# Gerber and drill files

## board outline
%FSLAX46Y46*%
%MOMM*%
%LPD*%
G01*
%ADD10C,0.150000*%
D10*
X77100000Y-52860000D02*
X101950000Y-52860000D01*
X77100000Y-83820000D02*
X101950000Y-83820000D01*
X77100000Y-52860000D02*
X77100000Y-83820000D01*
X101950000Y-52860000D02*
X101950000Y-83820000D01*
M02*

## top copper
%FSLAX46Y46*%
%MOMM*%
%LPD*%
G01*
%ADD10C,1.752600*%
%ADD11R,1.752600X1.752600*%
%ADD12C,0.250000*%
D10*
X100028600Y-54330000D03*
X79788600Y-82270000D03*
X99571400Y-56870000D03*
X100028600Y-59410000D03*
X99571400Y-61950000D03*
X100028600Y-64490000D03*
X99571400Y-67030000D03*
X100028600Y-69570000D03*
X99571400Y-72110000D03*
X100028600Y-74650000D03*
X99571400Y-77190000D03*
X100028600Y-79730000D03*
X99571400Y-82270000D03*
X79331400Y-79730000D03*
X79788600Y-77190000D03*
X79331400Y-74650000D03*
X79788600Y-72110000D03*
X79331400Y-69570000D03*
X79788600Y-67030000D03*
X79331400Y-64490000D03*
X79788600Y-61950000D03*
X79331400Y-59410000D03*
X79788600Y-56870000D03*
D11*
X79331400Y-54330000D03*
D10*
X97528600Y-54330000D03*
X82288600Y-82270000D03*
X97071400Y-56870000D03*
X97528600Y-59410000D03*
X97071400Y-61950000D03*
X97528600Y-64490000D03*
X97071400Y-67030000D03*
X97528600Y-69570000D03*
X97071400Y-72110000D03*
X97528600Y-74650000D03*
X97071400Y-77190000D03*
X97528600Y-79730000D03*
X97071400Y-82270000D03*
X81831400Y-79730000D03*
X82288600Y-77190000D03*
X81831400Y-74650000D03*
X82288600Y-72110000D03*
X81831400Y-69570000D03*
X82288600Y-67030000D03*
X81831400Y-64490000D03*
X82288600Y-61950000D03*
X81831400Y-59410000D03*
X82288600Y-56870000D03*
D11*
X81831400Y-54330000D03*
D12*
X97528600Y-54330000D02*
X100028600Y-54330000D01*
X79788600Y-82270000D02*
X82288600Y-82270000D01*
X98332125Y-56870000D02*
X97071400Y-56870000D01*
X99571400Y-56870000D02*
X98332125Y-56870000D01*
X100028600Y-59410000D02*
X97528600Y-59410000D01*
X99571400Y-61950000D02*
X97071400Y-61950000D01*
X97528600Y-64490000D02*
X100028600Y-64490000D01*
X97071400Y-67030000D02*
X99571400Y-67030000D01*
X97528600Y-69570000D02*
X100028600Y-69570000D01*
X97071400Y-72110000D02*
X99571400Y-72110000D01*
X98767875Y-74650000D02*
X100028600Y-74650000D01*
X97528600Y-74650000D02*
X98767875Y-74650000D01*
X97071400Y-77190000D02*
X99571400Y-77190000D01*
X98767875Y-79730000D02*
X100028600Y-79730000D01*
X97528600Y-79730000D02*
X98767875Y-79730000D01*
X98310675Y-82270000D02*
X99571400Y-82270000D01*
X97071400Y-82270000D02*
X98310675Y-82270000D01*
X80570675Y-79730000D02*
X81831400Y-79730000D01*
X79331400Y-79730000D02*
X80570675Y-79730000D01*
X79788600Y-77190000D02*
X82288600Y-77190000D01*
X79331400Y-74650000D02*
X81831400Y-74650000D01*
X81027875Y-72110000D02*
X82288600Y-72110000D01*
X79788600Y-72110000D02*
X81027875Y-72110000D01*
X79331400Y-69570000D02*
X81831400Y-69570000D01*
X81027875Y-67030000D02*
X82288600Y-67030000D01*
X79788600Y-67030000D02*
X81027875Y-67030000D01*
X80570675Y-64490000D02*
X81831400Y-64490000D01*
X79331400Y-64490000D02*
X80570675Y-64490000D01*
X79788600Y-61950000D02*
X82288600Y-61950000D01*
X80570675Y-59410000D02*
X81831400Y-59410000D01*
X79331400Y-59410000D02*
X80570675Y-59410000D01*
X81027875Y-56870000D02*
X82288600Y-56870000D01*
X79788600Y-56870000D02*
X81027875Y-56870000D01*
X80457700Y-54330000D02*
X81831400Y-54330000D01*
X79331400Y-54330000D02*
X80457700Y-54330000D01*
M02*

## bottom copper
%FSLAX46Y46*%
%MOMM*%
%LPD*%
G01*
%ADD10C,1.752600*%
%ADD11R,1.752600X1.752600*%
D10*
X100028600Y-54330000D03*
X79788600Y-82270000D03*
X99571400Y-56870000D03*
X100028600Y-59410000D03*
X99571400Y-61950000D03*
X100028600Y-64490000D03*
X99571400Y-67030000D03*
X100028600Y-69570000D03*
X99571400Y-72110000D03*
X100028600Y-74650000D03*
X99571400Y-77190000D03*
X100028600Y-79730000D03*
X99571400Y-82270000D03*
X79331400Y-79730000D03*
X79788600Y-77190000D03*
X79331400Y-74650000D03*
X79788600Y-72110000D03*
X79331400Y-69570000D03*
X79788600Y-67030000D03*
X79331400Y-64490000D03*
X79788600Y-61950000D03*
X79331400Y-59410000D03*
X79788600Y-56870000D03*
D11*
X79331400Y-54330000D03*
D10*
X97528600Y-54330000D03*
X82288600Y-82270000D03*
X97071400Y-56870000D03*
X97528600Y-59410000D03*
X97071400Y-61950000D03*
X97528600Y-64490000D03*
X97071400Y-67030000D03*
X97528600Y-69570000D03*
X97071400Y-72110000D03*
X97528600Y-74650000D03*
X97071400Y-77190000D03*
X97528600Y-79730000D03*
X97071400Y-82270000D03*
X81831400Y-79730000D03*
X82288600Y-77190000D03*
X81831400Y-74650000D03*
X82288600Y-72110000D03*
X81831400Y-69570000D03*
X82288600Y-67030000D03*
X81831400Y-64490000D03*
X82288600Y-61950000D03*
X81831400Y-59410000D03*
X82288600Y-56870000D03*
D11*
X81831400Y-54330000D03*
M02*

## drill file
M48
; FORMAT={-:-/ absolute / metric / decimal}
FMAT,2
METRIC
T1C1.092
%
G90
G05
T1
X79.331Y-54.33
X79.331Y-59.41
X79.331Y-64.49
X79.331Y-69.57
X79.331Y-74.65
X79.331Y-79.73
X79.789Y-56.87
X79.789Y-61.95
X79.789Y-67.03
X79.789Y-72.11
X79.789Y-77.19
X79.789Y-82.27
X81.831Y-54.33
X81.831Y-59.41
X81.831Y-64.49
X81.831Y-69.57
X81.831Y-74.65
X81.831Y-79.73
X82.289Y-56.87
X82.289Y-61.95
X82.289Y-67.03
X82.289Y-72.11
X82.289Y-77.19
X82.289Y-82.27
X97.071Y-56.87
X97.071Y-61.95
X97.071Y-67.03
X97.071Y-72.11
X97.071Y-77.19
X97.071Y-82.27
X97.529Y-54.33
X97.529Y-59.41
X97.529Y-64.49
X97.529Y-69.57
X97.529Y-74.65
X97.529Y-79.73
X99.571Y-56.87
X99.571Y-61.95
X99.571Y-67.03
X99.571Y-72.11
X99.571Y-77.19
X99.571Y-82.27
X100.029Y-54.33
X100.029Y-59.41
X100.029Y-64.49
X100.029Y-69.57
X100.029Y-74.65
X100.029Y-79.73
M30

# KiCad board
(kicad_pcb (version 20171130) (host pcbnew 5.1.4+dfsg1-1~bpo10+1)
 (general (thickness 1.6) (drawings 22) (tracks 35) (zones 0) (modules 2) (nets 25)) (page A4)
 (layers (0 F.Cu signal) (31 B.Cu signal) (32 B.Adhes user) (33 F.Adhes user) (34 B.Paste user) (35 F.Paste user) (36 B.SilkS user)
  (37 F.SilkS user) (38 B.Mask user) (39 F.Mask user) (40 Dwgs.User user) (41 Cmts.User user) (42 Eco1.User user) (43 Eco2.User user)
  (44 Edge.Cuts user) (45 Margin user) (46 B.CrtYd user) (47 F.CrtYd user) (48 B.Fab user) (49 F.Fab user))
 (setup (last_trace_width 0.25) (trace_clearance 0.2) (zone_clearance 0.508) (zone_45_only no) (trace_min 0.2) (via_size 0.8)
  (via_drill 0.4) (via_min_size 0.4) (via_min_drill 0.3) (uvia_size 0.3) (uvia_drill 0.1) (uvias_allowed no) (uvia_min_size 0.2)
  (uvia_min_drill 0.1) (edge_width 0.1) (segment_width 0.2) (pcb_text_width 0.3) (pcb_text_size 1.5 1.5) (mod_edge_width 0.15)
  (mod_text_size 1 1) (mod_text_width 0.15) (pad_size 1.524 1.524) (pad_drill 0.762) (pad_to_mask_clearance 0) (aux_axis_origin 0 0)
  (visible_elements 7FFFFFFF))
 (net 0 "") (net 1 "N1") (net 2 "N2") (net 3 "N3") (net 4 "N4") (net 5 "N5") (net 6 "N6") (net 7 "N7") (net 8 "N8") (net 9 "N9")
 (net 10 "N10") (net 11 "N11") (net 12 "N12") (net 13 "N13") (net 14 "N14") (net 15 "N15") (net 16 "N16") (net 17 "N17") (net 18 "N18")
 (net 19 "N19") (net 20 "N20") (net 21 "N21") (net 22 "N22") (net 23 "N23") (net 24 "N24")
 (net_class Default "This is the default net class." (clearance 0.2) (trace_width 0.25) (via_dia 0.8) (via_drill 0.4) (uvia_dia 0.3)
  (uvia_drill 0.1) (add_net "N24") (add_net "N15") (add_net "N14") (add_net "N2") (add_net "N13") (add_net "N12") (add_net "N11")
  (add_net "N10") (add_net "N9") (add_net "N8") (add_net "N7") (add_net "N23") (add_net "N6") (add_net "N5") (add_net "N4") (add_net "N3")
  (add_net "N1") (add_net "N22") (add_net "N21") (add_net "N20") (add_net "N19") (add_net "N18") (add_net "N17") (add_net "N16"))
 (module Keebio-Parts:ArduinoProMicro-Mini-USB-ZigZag (layer F.Cu) (at 89.68 68.3 270)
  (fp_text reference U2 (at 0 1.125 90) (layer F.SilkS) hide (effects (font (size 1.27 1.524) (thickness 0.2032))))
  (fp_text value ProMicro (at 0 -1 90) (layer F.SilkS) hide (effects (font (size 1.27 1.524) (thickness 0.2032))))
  (pad 24 thru_hole circle (at -13.97 -10.3486 270) (size 1.7526 1.7526) (drill 1.0922) (layers *.Cu *.SilkS *.Mask) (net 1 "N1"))
  (pad 12 thru_hole circle (at 13.97 9.8914 270) (size 1.7526 1.7526) (drill 1.0922) (layers *.Cu *.SilkS *.Mask) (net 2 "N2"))
  (pad 23 thru_hole circle (at -11.43 -9.8914 270) (size 1.7526 1.7526) (drill 1.0922) (layers *.Cu *.SilkS *.Mask) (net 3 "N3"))
  (pad 22 thru_hole circle (at -8.89 -10.3486 270) (size 1.7526 1.7526) (drill 1.0922) (layers *.Cu *.SilkS *.Mask) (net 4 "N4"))
  (pad 21 thru_hole circle (at -6.35 -9.8914 270) (size 1.7526 1.7526) (drill 1.0922) (layers *.Cu *.SilkS *.Mask) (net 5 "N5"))
  (pad 20 thru_hole circle (at -3.81 -10.3486 270) (size 1.7526 1.7526) (drill 1.0922) (layers *.Cu *.SilkS *.Mask) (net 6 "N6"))
  (pad 19 thru_hole circle (at -1.27 -9.8914 270) (size 1.7526 1.7526) (drill 1.0922) (layers *.Cu *.SilkS *.Mask) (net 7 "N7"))
  (pad 18 thru_hole circle (at 1.27 -10.3486 270) (size 1.7526 1.7526) (drill 1.0922) (layers *.Cu *.SilkS *.Mask) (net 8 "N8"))
  (pad 17 thru_hole circle (at 3.81 -9.8914 270) (size 1.7526 1.7526) (drill 1.0922) (layers *.Cu *.SilkS *.Mask) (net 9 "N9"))
  (pad 16 thru_hole circle (at 6.35 -10.3486 270) (size 1.7526 1.7526) (drill 1.0922) (layers *.Cu *.SilkS *.Mask) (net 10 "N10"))
  (pad 15 thru_hole circle (at 8.89 -9.8914 270) (size 1.7526 1.7526) (drill 1.0922) (layers *.Cu *.SilkS *.Mask) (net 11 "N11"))
  (pad 14 thru_hole circle (at 11.43 -10.3486 270) (size 1.7526 1.7526) (drill 1.0922) (layers *.Cu *.SilkS *.Mask) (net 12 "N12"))
  (pad 13 thru_hole circle (at 13.97 -9.8914 270) (size 1.7526 1.7526) (drill 1.0922) (layers *.Cu *.SilkS *.Mask) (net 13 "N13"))
  (pad 11 thru_hole circle (at 11.43 10.3486 270) (size 1.7526 1.7526) (drill 1.0922) (layers *.Cu *.SilkS *.Mask) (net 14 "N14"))
  (pad 10 thru_hole circle (at 8.89 9.8914 270) (size 1.7526 1.7526) (drill 1.0922) (layers *.Cu *.SilkS *.Mask) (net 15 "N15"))
  (pad 9 thru_hole circle (at 6.35 10.3486 270) (size 1.7526 1.7526) (drill 1.0922) (layers *.Cu *.SilkS *.Mask) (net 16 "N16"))
  (pad 8 thru_hole circle (at 3.81 9.8914 270) (size 1.7526 1.7526) (drill 1.0922) (layers *.Cu *.SilkS *.Mask) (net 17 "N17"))
  (pad 7 thru_hole circle (at 1.27 10.3486 270) (size 1.7526 1.7526) (drill 1.0922) (layers *.Cu *.SilkS *.Mask) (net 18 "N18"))
  (pad 6 thru_hole circle (at -1.27 9.8914 270) (size 1.7526 1.7526) (drill 1.0922) (layers *.Cu *.SilkS *.Mask) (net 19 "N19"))
  (pad 5 thru_hole circle (at -3.81 10.3486 270) (size 1.7526 1.7526) (drill 1.0922) (layers *.Cu *.SilkS *.Mask) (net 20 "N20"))
  (pad 4 thru_hole circle (at -6.35 9.8914 270) (size 1.7526 1.7526) (drill 1.0922) (layers *.Cu *.SilkS *.Mask) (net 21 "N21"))
  (pad 3 thru_hole circle (at -8.89 10.3486 270) (size 1.7526 1.7526) (drill 1.0922) (layers *.Cu *.SilkS *.Mask) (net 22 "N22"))
  (pad 2 thru_hole circle (at -11.43 9.8914 270) (size 1.7526 1.7526) (drill 1.0922) (layers *.Cu *.SilkS *.Mask) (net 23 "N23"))
  (pad 1 thru_hole rect (at -13.97 10.3486 270) (size 1.7526 1.7526) (drill 1.0922) (layers *.Cu *.SilkS *.Mask) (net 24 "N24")))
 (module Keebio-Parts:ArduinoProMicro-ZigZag (layer F.Cu) (at 89.68 68.3 270)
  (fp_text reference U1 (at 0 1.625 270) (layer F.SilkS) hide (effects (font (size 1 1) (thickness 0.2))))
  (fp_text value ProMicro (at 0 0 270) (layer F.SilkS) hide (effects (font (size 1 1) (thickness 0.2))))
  (pad 24 thru_hole circle (at -13.97 -7.8486 270) (size 1.7526 1.7526) (drill 1.0922) (layers *.Cu *.SilkS *.Mask) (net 1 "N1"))
  (pad 12 thru_hole circle (at 13.97 7.3914 270) (size 1.7526 1.7526) (drill 1.0922) (layers *.Cu *.SilkS *.Mask) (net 2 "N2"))
  (pad 23 thru_hole circle (at -11.43 -7.3914 270) (size 1.7526 1.7526) (drill 1.0922) (layers *.Cu *.SilkS *.Mask) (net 3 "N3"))
  (pad 22 thru_hole circle (at -8.89 -7.8486 270) (size 1.7526 1.7526) (drill 1.0922) (layers *.Cu *.SilkS *.Mask) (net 4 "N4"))
  (pad 21 thru_hole circle (at -6.35 -7.3914 270) (size 1.7526 1.7526) (drill 1.0922) (layers *.Cu *.SilkS *.Mask) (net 5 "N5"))
  (pad 20 thru_hole circle (at -3.81 -7.8486 270) (size 1.7526 1.7526) (drill 1.0922) (layers *.Cu *.SilkS *.Mask) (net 6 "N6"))
  (pad 19 thru_hole circle (at -1.27 -7.3914 270) (size 1.7526 1.7526) (drill 1.0922) (layers *.Cu *.SilkS *.Mask) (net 7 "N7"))
  (pad 18 thru_hole circle (at 1.27 -7.8486 270) (size 1.7526 1.7526) (drill 1.0922) (layers *.Cu *.SilkS *.Mask) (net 8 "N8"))
  (pad 17 thru_hole circle (at 3.81 -7.3914 270) (size 1.7526 1.7526) (drill 1.0922) (layers *.Cu *.SilkS *.Mask) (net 9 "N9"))
  (pad 16 thru_hole circle (at 6.35 -7.8486 270) (size 1.7526 1.7526) (drill 1.0922) (layers *.Cu *.SilkS *.Mask) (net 10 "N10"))
  (pad 15 thru_hole circle (at 8.89 -7.3914 270) (size 1.7526 1.7526) (drill 1.0922) (layers *.Cu *.SilkS *.Mask) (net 11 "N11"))
  (pad 14 thru_hole circle (at 11.43 -7.8486 270) (size 1.7526 1.7526) (drill 1.0922) (layers *.Cu *.SilkS *.Mask) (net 12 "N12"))
  (pad 13 thru_hole circle (at 13.97 -7.3914 270) (size 1.7526 1.7526) (drill 1.0922) (layers *.Cu *.SilkS *.Mask) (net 13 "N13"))
  (pad 11 thru_hole circle (at 11.43 7.8486 270) (size 1.7526 1.7526) (drill 1.0922) (layers *.Cu *.SilkS *.Mask) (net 14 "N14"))
  (pad 10 thru_hole circle (at 8.89 7.3914 270) (size 1.7526 1.7526) (drill 1.0922) (layers *.Cu *.SilkS *.Mask) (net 15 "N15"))
  (pad 9 thru_hole circle (at 6.35 7.8486 270) (size 1.7526 1.7526) (drill 1.0922) (layers *.Cu *.SilkS *.Mask) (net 16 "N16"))
  (pad 8 thru_hole circle (at 3.81 7.3914 270) (size 1.7526 1.7526) (drill 1.0922) (layers *.Cu *.SilkS *.Mask) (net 17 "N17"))
  (pad 7 thru_hole circle (at 1.27 7.8486 270) (size 1.7526 1.7526) (drill 1.0922) (layers *.Cu *.SilkS *.Mask) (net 18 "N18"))
  (pad 6 thru_hole circle (at -1.27 7.3914 270) (size 1.7526 1.7526) (drill 1.0922) (layers *.Cu *.SilkS *.Mask) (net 19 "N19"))
  (pad 5 thru_hole circle (at -3.81 7.8486 270) (size 1.7526 1.7526) (drill 1.0922) (layers *.Cu *.SilkS *.Mask) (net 20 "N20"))
  (pad 4 thru_hole circle (at -6.35 7.3914 270) (size 1.7526 1.7526) (drill 1.0922) (layers *.Cu *.SilkS *.Mask) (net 21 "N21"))
  (pad 3 thru_hole circle (at -8.89 7.8486 270) (size 1.7526 1.7526) (drill 1.0922) (layers *.Cu *.SilkS *.Mask) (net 22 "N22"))
  (pad 2 thru_hole circle (at -11.43 7.3914 270) (size 1.7526 1.7526) (drill 1.0922) (layers *.Cu *.SilkS *.Mask) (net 23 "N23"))
  (pad 1 thru_hole rect (at -13.97 7.8486 270) (size 1.7526 1.7526) (drill 1.0922) (layers *.Cu *.SilkS *.Mask) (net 24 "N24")))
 (gr_line (start 77.1 52.86) (end 101.95 52.86) (layer Edge.Cuts) (width 0.15))
 (gr_line (start 77.1 83.82) (end 101.95 83.82) (layer Edge.Cuts) (width 0.15))
 (gr_line (start 77.1 52.86) (end 77.1 83.82) (layer Edge.Cuts) (width 0.15))
 (gr_line (start 101.95 52.86) (end 101.95 83.82) (layer Edge.Cuts) (width 0.15))
 (segment (start 97.5286 54.33) (end 100.0286 54.33) (width 0.25) (layer F.Cu) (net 1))
 (segment (start 79.7886 82.27) (end 82.2886 82.27) (width 0.25) (layer F.Cu) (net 2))
 (segment (start 98.332125 56.87) (end 97.0714 56.87) (width 0.25) (layer F.Cu) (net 3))
 (segment (start 99.5714 56.87) (end 98.332125 56.87) (width 0.25) (layer F.Cu) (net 3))
 (segment (start 100.0286 59.41) (end 97.5286 59.41) (width 0.25) (layer F.Cu) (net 4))
 (segment (start 99.5714 61.95) (end 97.0714 61.95) (width 0.25) (layer F.Cu) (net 5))
 (segment (start 97.5286 64.49) (end 100.0286 64.49) (width 0.25) (layer F.Cu) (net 6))
 (segment (start 97.0714 67.03) (end 99.5714 67.03) (width 0.25) (layer F.Cu) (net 7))
 (segment (start 97.5286 69.57) (end 100.0286 69.57) (width 0.25) (layer F.Cu) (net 8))
 (segment (start 97.0714 72.11) (end 99.5714 72.11) (width 0.25) (layer F.Cu) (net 9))
 (segment (start 98.767875 74.65) (end 100.0286 74.65) (width 0.25) (layer F.Cu) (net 10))
 (segment (start 97.5286 74.65) (end 98.767875 74.65) (width 0.25) (layer F.Cu) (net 10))
 (segment (start 97.0714 77.19) (end 99.5714 77.19) (width 0.25) (layer F.Cu) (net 11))
 (segment (start 98.767875 79.73) (end 100.0286 79.73) (width 0.25) (layer F.Cu) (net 12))
 (segment (start 97.5286 79.73) (end 98.767875 79.73) (width 0.25) (layer F.Cu) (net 12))
 (segment (start 98.310675 82.27) (end 99.5714 82.27) (width 0.25) (layer F.Cu) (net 13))
 (segment (start 97.0714 82.27) (end 98.310675 82.27) (width 0.25) (layer F.Cu) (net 13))
 (segment (start 80.570675 79.73) (end 81.8314 79.73) (width 0.25) (layer F.Cu) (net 14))
 (segment (start 79.3314 79.73) (end 80.570675 79.73) (width 0.25) (layer F.Cu) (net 14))
 (segment (start 79.7886 77.19) (end 82.2886 77.19) (width 0.25) (layer F.Cu) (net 15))
 (segment (start 79.3314 74.65) (end 81.8314 74.65) (width 0.25) (layer F.Cu) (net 16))
 (segment (start 81.027875 72.11) (end 82.2886 72.11) (width 0.25) (layer F.Cu) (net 17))
 (segment (start 79.7886 72.11) (end 81.027875 72.11) (width 0.25) (layer F.Cu) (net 17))
 (segment (start 79.3314 69.57) (end 81.8314 69.57) (width 0.25) (layer F.Cu) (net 18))
 (segment (start 81.027875 67.03) (end 82.2886 67.03) (width 0.25) (layer F.Cu) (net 19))
 (segment (start 79.7886 67.03) (end 81.027875 67.03) (width 0.25) (layer F.Cu) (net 19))
 (segment (start 80.570675 64.49) (end 81.8314 64.49) (width 0.25) (layer F.Cu) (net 20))
 (segment (start 79.3314 64.49) (end 80.570675 64.49) (width 0.25) (layer F.Cu) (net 20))
 (segment (start 79.7886 61.95) (end 82.2886 61.95) (width 0.25) (layer F.Cu) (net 21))
 (segment (start 80.570675 59.41) (end 81.8314 59.41) (width 0.25) (layer F.Cu) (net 22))
 (segment (start 79.3314 59.41) (end 80.570675 59.41) (width 0.25) (layer F.Cu) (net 22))
 (segment (start 81.027875 56.87) (end 82.2886 56.87) (width 0.25) (layer F.Cu) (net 23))
 (segment (start 79.7886 56.87) (end 81.027875 56.87) (width 0.25) (layer F.Cu) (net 23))
 (segment (start 80.4577 54.33) (end 81.8314 54.33) (width 0.25) (layer F.Cu) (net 24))
 (segment (start 79.3314 54.33) (end 80.4577 54.33) (width 0.25) (layer F.Cu) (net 24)))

